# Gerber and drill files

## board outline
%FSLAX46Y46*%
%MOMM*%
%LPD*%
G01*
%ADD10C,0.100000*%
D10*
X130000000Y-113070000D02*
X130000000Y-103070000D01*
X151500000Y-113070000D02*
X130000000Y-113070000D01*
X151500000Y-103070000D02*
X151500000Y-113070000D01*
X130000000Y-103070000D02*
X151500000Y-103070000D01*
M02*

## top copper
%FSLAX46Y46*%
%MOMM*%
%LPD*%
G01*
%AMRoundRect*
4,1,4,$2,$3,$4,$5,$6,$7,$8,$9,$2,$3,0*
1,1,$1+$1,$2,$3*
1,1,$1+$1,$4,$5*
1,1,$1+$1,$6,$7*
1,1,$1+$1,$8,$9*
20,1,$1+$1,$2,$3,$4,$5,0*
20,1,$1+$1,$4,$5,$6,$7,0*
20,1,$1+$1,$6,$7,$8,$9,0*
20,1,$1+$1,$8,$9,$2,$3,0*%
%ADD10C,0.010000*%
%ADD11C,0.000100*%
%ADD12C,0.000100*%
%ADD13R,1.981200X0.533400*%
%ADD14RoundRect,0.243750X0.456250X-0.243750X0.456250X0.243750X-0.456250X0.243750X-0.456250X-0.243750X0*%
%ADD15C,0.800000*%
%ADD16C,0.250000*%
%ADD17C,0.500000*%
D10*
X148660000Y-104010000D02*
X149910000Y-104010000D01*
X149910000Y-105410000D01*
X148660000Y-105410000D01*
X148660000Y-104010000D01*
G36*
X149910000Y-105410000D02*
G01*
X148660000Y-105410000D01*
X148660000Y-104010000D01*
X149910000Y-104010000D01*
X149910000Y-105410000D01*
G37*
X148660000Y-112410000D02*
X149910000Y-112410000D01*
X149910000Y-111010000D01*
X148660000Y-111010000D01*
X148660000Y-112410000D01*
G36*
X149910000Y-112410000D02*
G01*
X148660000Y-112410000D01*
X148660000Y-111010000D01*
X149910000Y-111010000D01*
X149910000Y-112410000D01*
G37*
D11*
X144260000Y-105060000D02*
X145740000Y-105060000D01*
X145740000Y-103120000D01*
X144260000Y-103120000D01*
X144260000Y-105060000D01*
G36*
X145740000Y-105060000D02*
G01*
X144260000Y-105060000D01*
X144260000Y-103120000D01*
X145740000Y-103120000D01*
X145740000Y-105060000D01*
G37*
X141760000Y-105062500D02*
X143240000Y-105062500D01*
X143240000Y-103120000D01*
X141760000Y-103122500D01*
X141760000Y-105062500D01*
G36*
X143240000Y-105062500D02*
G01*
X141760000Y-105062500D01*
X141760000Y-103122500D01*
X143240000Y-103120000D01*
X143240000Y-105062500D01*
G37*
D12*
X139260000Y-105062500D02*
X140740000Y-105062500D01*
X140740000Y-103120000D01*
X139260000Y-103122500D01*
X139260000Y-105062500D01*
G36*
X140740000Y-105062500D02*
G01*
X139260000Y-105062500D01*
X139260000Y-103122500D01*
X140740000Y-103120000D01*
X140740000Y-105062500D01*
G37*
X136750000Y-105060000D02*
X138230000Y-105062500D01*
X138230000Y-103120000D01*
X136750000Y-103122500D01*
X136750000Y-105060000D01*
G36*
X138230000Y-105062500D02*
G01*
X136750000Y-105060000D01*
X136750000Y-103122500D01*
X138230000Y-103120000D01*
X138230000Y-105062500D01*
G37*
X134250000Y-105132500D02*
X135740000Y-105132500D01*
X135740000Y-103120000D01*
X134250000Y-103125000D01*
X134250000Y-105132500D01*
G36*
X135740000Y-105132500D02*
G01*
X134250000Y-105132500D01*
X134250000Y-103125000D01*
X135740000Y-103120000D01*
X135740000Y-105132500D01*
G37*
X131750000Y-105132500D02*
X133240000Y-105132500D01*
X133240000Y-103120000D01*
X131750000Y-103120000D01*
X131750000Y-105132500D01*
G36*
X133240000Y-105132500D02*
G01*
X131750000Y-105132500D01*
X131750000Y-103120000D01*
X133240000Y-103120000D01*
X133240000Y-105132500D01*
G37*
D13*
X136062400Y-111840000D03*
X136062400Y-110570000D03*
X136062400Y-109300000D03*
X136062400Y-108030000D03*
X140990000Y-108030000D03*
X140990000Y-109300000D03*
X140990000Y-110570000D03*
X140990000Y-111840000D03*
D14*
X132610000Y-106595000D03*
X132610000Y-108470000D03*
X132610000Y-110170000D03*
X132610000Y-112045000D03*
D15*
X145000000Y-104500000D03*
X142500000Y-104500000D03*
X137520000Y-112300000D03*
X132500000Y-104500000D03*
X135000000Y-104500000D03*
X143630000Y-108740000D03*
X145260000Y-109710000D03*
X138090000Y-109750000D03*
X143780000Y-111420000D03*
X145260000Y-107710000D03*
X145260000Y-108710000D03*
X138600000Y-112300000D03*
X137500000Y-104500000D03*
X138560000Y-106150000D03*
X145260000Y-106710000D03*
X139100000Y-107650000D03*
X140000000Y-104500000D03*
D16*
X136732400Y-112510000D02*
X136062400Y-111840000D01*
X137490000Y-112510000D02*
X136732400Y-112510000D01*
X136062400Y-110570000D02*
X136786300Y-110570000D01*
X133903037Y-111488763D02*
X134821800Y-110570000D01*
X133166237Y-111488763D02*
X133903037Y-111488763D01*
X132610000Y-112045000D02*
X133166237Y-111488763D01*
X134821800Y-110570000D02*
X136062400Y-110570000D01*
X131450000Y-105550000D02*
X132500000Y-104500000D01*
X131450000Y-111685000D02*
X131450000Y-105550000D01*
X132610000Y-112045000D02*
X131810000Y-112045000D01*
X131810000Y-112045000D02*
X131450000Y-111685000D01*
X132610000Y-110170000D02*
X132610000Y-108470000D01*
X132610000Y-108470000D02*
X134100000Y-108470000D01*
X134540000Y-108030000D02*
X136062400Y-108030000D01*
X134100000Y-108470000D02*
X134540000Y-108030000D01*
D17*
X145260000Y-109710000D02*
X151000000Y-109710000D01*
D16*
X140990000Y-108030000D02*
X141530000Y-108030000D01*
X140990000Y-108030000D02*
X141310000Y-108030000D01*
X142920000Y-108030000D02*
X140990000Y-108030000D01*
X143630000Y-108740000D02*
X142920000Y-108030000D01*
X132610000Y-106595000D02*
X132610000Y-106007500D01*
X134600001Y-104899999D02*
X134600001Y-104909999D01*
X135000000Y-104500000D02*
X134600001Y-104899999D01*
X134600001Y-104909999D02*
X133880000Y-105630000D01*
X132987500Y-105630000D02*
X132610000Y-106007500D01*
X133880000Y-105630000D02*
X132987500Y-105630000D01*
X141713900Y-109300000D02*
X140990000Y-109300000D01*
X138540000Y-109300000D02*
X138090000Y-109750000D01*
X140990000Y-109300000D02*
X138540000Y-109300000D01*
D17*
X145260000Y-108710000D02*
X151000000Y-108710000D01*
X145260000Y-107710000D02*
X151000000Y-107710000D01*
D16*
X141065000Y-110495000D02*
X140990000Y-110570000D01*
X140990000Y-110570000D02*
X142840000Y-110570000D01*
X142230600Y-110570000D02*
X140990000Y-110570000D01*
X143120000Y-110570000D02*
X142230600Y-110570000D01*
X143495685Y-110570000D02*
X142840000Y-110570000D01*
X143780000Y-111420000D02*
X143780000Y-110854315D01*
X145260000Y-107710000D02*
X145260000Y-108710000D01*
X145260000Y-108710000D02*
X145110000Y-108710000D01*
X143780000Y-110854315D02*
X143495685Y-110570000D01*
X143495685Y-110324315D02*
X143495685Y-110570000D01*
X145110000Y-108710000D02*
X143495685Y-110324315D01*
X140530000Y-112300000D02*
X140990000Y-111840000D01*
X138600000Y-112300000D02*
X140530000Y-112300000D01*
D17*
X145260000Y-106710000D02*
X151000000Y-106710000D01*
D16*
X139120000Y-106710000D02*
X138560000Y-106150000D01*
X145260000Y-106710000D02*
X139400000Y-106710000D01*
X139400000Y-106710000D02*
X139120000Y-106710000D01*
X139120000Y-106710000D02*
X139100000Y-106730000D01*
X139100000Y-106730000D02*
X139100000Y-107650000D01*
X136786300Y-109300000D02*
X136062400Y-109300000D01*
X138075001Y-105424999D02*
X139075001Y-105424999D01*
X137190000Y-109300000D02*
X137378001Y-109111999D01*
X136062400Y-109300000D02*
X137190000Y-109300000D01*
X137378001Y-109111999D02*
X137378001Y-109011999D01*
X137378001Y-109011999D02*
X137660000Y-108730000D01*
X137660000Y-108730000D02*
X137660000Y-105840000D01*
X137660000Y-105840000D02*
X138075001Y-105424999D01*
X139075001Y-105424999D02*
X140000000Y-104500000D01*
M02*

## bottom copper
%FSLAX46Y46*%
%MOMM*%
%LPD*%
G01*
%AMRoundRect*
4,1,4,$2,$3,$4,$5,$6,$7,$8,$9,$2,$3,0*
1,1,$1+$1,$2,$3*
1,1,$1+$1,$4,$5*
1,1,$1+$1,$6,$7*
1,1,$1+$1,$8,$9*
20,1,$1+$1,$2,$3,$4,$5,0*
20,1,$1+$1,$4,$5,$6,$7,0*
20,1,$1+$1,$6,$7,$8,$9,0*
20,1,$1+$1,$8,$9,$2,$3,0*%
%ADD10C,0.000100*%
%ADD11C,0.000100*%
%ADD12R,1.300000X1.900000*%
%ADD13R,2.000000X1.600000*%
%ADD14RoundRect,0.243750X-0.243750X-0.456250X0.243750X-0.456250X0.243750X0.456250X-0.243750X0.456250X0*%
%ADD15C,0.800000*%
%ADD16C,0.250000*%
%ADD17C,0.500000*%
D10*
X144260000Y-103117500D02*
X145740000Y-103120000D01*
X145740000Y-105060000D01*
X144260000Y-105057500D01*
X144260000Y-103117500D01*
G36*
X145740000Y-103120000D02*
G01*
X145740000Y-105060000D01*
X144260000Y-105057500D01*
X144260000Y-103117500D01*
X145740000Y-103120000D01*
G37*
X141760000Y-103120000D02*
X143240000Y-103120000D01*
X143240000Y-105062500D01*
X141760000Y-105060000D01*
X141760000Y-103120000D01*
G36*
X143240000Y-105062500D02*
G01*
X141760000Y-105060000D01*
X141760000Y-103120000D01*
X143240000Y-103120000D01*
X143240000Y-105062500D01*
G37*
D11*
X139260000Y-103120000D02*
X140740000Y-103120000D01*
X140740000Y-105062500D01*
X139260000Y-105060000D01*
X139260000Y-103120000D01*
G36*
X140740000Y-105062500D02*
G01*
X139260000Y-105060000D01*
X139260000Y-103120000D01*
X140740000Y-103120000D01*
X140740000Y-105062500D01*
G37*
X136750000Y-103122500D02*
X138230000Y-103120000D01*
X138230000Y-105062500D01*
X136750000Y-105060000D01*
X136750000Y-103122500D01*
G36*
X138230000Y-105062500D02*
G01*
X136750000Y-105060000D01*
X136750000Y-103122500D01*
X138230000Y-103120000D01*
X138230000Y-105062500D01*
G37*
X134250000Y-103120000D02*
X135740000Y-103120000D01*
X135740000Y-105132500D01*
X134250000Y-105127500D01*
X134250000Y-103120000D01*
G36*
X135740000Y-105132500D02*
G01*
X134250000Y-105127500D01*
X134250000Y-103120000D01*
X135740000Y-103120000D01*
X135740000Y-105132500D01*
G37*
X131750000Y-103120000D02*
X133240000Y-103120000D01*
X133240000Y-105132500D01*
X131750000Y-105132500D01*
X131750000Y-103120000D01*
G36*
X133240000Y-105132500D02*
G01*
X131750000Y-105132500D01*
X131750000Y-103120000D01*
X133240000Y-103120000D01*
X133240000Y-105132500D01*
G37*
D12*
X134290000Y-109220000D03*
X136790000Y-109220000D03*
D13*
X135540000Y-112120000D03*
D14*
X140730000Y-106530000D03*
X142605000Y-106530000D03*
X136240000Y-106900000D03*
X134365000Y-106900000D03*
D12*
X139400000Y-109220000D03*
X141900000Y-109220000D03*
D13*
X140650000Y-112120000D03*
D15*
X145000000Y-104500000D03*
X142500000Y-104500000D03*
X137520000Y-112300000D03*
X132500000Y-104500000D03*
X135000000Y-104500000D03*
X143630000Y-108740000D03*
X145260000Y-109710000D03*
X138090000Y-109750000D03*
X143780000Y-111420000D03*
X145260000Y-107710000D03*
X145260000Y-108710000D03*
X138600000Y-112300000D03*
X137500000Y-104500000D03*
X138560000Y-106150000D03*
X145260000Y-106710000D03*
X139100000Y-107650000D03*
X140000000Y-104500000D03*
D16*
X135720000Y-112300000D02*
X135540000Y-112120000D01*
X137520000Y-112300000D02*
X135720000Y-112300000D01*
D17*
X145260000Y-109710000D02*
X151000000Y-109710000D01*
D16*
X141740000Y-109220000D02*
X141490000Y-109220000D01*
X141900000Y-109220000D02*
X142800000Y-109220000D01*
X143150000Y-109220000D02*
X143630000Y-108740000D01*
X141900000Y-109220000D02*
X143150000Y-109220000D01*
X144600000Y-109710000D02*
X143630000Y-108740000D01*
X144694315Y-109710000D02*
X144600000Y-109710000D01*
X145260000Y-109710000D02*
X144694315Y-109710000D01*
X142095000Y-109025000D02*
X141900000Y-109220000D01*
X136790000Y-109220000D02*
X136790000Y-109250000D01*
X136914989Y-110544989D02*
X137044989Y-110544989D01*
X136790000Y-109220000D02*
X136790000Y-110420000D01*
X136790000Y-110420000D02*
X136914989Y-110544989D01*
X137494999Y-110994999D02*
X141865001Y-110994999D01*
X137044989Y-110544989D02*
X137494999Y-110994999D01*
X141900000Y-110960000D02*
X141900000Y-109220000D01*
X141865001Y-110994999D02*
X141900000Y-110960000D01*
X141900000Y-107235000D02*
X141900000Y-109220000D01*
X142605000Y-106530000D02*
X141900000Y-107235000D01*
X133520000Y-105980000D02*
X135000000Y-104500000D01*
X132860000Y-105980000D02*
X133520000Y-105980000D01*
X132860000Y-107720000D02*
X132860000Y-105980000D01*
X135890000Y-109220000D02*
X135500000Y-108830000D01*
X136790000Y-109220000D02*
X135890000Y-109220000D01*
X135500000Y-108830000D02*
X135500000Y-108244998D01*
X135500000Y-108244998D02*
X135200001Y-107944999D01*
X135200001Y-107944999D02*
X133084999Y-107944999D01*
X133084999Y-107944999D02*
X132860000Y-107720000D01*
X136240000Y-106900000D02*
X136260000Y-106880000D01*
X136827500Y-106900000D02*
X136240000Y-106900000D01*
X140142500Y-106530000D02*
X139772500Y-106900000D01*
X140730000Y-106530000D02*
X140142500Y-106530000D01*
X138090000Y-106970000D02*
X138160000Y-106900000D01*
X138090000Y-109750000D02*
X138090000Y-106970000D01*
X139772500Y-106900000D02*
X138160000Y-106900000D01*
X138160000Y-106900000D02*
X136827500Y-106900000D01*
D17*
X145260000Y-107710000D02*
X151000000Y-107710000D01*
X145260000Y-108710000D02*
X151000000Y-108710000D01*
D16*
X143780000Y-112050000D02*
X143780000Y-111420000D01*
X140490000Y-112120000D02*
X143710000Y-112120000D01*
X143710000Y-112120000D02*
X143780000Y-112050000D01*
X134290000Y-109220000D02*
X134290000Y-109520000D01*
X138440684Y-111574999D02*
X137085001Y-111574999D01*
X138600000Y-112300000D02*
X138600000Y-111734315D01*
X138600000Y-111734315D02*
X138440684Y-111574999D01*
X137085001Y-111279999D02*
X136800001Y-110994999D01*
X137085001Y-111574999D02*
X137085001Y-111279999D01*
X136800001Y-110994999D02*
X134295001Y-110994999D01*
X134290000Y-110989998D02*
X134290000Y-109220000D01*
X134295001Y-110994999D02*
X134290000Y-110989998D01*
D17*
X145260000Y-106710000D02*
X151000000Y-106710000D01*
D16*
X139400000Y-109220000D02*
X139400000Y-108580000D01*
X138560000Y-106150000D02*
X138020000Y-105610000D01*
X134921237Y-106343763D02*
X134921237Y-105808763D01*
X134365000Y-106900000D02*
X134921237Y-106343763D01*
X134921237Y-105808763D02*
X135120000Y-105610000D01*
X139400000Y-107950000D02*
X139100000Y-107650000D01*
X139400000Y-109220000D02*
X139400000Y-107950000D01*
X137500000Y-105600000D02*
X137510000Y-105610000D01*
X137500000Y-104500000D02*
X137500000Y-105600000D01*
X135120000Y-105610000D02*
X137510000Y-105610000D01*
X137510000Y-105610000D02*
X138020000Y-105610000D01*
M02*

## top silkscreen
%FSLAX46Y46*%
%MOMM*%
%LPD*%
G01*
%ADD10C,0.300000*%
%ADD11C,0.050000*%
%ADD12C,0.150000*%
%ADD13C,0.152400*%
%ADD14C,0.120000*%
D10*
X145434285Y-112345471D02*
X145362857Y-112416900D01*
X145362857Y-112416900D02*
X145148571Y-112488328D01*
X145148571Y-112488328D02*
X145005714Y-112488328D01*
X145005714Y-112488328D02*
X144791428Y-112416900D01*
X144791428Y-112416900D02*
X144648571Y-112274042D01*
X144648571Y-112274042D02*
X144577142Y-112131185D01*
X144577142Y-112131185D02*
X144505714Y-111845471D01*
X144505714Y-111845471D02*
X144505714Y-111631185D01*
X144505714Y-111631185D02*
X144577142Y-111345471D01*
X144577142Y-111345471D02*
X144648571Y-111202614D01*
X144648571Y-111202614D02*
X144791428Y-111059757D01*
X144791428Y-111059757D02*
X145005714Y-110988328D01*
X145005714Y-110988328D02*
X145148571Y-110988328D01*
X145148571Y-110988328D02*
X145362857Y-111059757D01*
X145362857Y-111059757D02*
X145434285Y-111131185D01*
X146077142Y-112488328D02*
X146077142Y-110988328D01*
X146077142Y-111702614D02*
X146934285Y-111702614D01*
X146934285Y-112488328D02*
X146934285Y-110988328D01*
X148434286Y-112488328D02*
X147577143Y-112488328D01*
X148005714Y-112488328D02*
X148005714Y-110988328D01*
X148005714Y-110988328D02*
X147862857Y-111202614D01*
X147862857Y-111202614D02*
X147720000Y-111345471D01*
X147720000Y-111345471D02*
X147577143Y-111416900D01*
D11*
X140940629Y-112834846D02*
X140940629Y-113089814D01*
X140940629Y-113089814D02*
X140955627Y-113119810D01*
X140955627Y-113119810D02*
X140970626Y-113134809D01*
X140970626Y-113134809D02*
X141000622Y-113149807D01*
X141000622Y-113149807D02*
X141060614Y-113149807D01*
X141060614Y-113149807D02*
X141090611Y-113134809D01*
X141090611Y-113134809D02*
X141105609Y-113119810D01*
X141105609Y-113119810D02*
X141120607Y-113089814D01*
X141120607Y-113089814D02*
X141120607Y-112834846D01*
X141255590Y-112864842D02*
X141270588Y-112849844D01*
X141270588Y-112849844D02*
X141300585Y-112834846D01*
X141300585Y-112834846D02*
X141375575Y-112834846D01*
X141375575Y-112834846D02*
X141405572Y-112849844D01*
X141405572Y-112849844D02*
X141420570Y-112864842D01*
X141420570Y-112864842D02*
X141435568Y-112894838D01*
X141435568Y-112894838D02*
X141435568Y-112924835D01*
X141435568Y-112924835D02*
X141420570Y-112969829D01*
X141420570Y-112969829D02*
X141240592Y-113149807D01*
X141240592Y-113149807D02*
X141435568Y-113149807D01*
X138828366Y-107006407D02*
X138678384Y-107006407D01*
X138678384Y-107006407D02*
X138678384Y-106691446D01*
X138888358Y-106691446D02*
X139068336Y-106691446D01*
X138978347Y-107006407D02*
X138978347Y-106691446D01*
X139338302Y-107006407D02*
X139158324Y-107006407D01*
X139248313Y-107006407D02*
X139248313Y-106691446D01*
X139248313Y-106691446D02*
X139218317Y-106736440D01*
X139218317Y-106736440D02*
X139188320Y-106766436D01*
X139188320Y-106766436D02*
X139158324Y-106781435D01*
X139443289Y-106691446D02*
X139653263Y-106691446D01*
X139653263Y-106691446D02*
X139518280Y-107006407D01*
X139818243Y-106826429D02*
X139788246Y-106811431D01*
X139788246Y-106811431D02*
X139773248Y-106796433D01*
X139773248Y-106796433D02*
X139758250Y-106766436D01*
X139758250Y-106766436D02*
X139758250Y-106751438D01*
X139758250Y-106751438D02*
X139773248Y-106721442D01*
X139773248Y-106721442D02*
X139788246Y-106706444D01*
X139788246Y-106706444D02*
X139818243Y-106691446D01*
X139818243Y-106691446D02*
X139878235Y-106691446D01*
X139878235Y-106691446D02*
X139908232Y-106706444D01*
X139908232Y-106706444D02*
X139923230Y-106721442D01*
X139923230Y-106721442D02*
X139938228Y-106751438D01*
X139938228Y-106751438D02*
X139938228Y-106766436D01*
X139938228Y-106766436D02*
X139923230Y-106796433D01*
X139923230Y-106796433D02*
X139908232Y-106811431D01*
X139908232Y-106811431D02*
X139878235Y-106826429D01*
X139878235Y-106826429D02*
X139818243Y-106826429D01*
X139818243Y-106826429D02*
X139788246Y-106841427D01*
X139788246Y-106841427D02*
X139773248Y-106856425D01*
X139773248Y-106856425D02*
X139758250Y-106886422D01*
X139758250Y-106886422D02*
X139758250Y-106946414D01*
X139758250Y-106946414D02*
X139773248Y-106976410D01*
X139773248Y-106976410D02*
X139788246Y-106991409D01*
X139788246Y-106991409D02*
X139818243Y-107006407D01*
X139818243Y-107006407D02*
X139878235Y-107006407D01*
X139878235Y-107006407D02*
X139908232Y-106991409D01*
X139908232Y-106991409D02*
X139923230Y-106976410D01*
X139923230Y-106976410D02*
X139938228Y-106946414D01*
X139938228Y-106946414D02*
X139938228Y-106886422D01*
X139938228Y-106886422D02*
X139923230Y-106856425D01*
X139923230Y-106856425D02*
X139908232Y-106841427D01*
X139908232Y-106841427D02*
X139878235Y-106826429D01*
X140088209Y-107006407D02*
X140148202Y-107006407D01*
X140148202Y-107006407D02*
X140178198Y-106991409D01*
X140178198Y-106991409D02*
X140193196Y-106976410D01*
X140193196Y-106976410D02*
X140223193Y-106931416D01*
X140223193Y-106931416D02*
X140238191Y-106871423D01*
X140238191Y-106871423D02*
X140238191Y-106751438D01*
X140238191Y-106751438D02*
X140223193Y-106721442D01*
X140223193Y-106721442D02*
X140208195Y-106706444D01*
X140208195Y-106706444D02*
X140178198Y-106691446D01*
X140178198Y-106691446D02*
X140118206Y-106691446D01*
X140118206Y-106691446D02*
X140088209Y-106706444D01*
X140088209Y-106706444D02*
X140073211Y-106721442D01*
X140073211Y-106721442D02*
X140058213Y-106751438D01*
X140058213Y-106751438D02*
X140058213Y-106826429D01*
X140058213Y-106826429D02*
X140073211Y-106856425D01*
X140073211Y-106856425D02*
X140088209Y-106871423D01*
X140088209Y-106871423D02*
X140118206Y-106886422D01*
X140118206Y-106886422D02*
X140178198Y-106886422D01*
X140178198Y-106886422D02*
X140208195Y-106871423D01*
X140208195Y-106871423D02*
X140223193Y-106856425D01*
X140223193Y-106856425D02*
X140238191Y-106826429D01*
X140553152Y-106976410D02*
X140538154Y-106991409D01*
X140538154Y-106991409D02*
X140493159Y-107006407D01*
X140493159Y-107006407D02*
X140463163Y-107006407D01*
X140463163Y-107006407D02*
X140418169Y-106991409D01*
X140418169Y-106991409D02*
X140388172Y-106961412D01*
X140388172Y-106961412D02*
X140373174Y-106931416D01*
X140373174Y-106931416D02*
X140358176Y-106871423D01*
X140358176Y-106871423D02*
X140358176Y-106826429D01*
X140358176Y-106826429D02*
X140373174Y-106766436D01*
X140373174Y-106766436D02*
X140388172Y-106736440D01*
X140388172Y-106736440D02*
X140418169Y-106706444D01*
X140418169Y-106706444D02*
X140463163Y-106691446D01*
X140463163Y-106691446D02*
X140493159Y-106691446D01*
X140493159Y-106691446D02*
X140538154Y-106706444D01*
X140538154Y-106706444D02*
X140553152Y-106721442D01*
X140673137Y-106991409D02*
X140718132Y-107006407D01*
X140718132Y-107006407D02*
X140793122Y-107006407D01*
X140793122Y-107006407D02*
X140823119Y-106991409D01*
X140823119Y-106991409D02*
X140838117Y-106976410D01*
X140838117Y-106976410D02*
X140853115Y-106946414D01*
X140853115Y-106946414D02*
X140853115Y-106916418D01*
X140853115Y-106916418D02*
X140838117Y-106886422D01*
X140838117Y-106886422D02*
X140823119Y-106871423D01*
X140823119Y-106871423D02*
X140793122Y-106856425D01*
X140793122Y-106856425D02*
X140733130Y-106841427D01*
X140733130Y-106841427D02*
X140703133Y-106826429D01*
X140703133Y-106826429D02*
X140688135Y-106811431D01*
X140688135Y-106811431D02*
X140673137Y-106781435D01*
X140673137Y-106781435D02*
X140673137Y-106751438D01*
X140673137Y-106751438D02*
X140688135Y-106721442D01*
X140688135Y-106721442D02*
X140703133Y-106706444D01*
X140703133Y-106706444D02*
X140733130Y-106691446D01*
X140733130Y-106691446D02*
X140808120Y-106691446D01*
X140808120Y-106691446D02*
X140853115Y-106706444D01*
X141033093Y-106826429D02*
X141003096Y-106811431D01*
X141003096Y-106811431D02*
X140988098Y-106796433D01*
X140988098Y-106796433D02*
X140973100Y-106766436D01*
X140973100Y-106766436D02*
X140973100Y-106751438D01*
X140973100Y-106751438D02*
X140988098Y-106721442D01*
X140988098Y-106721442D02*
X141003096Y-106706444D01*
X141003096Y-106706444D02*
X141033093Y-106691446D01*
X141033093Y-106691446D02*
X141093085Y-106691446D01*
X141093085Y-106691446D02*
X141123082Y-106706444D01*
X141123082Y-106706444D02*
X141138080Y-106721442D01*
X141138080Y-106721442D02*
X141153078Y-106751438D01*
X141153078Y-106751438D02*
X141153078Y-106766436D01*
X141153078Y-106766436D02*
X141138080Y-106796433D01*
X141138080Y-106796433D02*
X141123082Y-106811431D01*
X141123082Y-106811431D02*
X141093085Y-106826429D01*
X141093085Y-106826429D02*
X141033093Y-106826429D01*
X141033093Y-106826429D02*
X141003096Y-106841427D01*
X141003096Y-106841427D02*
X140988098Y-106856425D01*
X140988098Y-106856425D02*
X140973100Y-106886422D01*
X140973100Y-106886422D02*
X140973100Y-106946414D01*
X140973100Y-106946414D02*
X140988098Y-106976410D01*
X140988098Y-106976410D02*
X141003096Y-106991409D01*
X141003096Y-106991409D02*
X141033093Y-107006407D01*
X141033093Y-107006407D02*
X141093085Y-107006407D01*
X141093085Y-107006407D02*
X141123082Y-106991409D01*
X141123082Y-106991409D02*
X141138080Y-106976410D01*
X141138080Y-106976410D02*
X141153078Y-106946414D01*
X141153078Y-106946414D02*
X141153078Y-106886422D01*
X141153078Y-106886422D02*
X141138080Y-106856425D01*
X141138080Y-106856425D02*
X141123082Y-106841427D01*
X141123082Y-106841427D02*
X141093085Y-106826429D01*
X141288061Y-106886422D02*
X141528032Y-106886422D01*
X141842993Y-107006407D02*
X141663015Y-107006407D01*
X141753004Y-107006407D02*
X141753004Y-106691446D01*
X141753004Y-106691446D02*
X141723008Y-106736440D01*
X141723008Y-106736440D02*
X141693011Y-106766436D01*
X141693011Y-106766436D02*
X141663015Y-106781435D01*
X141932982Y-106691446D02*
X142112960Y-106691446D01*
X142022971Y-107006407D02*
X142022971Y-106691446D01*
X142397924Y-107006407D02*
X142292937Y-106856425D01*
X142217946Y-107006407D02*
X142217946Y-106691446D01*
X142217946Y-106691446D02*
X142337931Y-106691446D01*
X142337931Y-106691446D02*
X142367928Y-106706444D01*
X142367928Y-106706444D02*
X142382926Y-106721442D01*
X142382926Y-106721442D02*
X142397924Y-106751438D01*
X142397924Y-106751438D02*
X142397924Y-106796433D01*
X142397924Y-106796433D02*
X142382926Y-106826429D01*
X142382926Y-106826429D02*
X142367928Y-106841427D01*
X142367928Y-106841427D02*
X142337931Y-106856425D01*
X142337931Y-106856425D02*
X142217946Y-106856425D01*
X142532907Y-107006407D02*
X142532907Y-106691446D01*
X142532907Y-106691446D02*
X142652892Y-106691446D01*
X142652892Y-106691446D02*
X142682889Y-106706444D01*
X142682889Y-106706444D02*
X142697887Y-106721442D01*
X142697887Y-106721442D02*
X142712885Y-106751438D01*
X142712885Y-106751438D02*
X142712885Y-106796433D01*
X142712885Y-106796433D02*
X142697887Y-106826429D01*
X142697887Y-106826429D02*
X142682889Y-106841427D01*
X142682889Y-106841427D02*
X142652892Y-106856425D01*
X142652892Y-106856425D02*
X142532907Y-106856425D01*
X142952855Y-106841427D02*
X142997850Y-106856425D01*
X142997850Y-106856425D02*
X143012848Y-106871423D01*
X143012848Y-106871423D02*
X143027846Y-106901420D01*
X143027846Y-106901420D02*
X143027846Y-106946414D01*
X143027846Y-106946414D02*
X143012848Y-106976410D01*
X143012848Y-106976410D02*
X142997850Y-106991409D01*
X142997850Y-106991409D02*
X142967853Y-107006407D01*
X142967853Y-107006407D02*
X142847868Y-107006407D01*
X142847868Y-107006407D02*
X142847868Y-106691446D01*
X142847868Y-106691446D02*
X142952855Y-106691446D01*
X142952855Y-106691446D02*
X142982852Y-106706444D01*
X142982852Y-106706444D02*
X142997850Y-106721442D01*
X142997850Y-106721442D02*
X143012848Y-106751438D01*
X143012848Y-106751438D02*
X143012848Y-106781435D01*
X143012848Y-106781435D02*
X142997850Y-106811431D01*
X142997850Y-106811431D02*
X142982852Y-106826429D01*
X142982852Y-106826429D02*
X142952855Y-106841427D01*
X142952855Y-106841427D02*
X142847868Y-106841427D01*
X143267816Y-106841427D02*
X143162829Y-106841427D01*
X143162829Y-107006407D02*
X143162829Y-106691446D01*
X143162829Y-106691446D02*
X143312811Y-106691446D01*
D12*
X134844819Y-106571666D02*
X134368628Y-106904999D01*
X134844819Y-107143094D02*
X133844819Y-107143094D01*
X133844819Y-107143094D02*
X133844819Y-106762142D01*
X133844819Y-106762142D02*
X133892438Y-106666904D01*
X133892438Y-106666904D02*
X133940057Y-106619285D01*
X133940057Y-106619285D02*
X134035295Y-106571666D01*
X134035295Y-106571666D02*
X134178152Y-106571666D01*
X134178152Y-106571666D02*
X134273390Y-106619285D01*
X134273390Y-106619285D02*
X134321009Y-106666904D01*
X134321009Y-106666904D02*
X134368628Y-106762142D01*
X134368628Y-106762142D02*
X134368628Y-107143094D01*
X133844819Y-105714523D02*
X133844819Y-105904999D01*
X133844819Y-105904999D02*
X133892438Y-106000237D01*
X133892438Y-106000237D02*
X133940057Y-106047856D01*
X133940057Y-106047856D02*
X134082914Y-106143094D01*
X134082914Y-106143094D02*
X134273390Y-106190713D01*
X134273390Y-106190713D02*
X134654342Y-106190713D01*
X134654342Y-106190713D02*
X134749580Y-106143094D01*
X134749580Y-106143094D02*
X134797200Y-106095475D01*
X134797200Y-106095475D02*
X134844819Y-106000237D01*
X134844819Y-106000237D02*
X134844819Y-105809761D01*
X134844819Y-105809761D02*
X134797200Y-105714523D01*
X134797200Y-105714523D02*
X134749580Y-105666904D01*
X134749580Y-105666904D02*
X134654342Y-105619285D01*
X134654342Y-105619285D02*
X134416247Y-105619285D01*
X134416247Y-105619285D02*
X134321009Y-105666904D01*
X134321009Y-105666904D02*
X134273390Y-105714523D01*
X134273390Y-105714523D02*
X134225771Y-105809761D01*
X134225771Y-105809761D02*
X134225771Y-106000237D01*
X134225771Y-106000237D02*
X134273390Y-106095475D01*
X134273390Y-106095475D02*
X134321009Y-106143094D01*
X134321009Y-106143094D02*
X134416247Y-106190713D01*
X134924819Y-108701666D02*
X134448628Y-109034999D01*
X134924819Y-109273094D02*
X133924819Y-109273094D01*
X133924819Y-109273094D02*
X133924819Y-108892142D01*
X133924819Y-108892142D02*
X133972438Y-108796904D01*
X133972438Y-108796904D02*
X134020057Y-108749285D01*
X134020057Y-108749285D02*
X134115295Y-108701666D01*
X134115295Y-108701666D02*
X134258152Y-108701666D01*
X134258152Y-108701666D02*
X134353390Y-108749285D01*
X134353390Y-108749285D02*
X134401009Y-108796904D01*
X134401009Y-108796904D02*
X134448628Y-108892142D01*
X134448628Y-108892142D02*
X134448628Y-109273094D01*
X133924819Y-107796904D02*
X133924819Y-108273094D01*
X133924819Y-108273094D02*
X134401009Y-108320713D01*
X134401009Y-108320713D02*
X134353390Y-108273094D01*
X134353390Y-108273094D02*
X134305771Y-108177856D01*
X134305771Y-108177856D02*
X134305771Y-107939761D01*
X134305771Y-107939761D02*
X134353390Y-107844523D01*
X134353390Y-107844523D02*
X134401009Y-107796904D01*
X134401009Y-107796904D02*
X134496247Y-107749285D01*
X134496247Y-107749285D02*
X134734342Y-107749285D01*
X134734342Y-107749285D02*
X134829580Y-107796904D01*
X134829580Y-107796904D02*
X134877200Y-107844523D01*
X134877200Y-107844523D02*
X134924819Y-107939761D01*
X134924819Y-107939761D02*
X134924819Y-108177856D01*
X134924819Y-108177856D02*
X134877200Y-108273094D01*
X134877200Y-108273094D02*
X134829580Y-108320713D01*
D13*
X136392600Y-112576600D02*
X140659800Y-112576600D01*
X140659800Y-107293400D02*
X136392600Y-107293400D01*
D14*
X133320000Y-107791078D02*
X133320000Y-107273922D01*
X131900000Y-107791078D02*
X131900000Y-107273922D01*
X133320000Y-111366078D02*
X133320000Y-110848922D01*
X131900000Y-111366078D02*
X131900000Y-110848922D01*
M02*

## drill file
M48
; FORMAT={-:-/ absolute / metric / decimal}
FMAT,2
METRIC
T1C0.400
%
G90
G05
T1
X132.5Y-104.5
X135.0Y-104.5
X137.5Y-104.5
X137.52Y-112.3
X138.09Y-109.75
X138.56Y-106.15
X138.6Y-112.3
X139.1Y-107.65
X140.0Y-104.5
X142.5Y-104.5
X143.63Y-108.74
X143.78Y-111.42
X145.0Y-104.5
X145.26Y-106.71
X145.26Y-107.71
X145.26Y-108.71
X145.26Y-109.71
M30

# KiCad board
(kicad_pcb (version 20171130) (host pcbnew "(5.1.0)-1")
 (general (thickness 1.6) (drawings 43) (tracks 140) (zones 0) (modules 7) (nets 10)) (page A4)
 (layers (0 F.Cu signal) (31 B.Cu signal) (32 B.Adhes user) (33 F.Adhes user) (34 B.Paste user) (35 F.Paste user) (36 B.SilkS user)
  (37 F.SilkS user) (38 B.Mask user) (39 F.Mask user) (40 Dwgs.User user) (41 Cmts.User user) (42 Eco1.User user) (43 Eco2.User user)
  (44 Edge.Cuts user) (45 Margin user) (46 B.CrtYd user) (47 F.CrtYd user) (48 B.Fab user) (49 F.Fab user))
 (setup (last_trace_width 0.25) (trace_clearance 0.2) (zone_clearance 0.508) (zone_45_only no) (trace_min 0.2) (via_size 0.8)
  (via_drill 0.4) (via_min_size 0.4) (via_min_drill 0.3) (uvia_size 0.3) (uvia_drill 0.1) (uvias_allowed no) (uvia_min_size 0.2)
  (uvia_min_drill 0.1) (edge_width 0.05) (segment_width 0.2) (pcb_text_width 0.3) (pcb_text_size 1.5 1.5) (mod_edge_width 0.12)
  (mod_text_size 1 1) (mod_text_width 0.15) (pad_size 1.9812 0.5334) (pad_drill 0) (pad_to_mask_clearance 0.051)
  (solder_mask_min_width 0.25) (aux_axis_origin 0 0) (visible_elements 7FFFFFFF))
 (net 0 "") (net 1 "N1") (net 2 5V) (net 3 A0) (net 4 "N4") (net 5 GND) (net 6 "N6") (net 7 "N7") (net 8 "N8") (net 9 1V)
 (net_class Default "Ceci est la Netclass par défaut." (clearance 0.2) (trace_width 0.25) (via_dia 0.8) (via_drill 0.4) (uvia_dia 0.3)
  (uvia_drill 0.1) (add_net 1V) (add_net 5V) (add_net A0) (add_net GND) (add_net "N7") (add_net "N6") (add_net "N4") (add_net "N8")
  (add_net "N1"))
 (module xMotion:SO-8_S (layer F.Cu) (at 138.5262 109.935 180)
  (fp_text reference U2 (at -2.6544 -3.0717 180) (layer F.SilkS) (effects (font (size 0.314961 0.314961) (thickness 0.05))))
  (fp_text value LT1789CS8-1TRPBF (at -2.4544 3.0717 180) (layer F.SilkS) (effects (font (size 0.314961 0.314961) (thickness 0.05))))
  (fp_line (start 2.1336 -2.6416) (end -2.1336 -2.6416) (layer F.SilkS) (width 0.1524))
  (fp_line (start -2.1336 2.6416) (end 2.1336 2.6416) (layer F.SilkS) (width 0.1524))
  (pad 8 smd rect (at 2.4638 -1.905 180) (size 1.9812 0.5334) (layers F.Cu F.Paste F.Mask) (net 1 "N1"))
  (pad 7 smd rect (at 2.4638 -0.635 180) (size 1.9812 0.5334) (layers F.Cu F.Paste F.Mask) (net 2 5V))
  (pad 6 smd rect (at 2.4638 0.635 180) (size 1.9812 0.5334) (layers F.Cu F.Paste F.Mask) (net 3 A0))
  (pad 5 smd rect (at 2.4638 1.905 180) (size 1.9812 0.5334) (layers F.Cu F.Paste F.Mask) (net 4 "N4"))
  (pad 4 smd rect (at -2.4638 1.905 180) (size 1.9812 0.5334) (layers F.Cu F.Paste F.Mask) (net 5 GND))
  (pad 3 smd rect (at -2.4638 0.635 180) (size 1.9812 0.5334) (layers F.Cu F.Paste F.Mask) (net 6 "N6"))
  (pad 2 smd rect (at -2.4638 -0.635 180) (size 1.9812 0.5334) (layers F.Cu F.Paste F.Mask) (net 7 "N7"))
  (pad 1 smd rect (at -2.4638 -1.905 180) (size 1.9812 0.5334) (layers F.Cu F.Paste F.Mask) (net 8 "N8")))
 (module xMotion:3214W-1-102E (layer B.Cu) (at 135.54 112.12 90)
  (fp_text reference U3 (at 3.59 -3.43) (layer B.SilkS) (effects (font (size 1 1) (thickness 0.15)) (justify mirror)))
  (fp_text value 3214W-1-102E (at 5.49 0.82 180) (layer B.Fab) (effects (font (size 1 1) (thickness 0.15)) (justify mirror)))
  (pad 3 smd rect (at 2.9 -1.25 90) (size 1.9 1.3) (layers B.Cu B.Paste B.Mask) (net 8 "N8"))
  (pad 2 smd rect (at 2.9 1.25 90) (size 1.9 1.3) (layers B.Cu B.Paste B.Mask) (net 5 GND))
  (pad 1 smd rect (at 0 0 90) (size 1.6 2) (layers B.Cu B.Paste B.Mask) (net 1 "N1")))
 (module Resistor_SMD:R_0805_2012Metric (layer F.Cu) (at 132.61 107.5325 90)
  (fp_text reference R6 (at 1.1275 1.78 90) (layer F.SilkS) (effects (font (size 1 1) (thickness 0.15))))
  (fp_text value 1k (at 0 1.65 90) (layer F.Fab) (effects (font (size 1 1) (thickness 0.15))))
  (fp_line (start -0.258578 0.71) (end 0.258578 0.71) (layer F.SilkS) (width 0.12))
  (fp_line (start -0.258578 -0.71) (end 0.258578 -0.71) (layer F.SilkS) (width 0.12))
  (pad 2 smd roundrect (at 0.9375 0 90) (size 0.975 1.4) (layers F.Cu F.Paste F.Mask) (roundrect_rratio 0.25) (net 5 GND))
  (pad 1 smd roundrect (at -0.9375 0 90) (size 0.975 1.4) (layers F.Cu F.Paste F.Mask) (roundrect_rratio 0.25) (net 4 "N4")))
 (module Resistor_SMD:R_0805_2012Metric (layer F.Cu) (at 132.61 111.1075 90)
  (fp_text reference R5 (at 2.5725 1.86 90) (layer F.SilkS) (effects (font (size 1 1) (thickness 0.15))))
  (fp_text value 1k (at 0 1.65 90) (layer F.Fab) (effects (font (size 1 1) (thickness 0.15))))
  (fp_line (start -0.258578 0.71) (end 0.258578 0.71) (layer F.SilkS) (width 0.12))
  (fp_line (start -0.258578 -0.71) (end 0.258578 -0.71) (layer F.SilkS) (width 0.12))
  (pad 2 smd roundrect (at 0.9375 0 90) (size 0.975 1.4) (layers F.Cu F.Paste F.Mask) (roundrect_rratio 0.25) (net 4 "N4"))
  (pad 1 smd roundrect (at -0.9375 0 90) (size 0.975 1.4) (layers F.Cu F.Paste F.Mask) (roundrect_rratio 0.25) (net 2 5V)))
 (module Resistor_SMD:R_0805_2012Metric (layer B.Cu) (at 141.6675 106.53)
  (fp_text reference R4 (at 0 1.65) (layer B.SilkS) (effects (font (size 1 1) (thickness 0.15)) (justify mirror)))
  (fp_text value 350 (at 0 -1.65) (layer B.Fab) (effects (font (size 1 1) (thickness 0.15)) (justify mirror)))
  (pad 1 smd roundrect (at -0.9375 0) (size 0.975 1.4) (layers B.Cu B.Paste B.Mask) (roundrect_rratio 0.25) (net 6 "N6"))
  (pad 2 smd roundrect (at 0.9375 0) (size 0.975 1.4) (layers B.Cu B.Paste B.Mask) (roundrect_rratio 0.25) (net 5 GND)))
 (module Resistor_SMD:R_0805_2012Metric (layer B.Cu) (at 135.3025 106.9)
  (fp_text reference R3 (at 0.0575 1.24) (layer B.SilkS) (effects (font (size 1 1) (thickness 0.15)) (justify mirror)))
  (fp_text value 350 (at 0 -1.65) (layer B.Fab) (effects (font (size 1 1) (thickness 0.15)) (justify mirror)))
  (pad 2 smd roundrect (at 0.9375 0) (size 0.975 1.4) (layers B.Cu B.Paste B.Mask) (roundrect_rratio 0.25) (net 6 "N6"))
  (pad 1 smd roundrect (at -0.9375 0) (size 0.975 1.4) (layers B.Cu B.Paste B.Mask) (roundrect_rratio 0.25) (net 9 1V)))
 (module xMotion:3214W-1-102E (layer B.Cu) (at 140.65 112.12 90)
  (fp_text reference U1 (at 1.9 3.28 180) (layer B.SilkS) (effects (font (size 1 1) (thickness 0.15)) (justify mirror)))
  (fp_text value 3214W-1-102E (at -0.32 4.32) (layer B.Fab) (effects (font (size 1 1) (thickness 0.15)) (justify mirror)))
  (pad 3 smd rect (at 2.9 -1.25 90) (size 1.9 1.3) (layers B.Cu B.Paste B.Mask) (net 9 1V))
  (pad 2 smd rect (at 2.9 1.25 90) (size 1.9 1.3) (layers B.Cu B.Paste B.Mask) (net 5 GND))
  (pad 1 smd rect (at 0 0 90) (size 1.6 2) (layers B.Cu B.Paste B.Mask) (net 7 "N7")))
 (gr_poly (pts (xy 148.66 104.01) (xy 149.91 104.01) (xy 149.91 105.41) (xy 148.66 105.41)) (layer F.Cu) (width 0.01))
 (gr_poly (pts (xy 148.66 112.41) (xy 149.91 112.41) (xy 149.91 111.01) (xy 148.66 111.01)) (layer F.Cu) (width 0.01))
 (gr_poly (pts (xy 144.26 103.1175) (xy 145.74 103.12) (xy 145.74 105.06) (xy 144.26 105.0575)) (layer B.Cu) (width 0.0001))
 (gr_poly (pts (xy 144.26 105.06) (xy 145.74 105.06) (xy 145.74 103.12) (xy 144.26 103.12)) (layer F.Cu) (width 0.0001))
 (gr_poly (pts (xy 141.76 103.12) (xy 143.24 103.12) (xy 143.24 105.0625) (xy 141.76 105.06)) (layer B.Cu) (width 0.0001))
 (gr_poly (pts (xy 141.76 105.0625) (xy 143.24 105.0625) (xy 143.24 103.12) (xy 141.76 103.1225)) (layer F.Cu) (width 0.0001))
 (gr_poly (pts (xy 139.26 103.12) (xy 140.74 103.12) (xy 140.74 105.0625) (xy 139.26 105.06)) (layer B.Cu) (width 0.0001))
 (gr_poly (pts (xy 139.26 105.0625) (xy 140.74 105.0625) (xy 140.74 103.12) (xy 139.26 103.1225)) (layer F.Cu) (width 0.0001))
 (gr_poly (pts (xy 136.75 103.1225) (xy 138.23 103.12) (xy 138.23 105.0625) (xy 136.75 105.06)) (layer B.Cu) (width 0.0001))
 (gr_poly (pts (xy 136.75 105.06) (xy 138.23 105.0625) (xy 138.23 103.12) (xy 136.75 103.1225)) (layer F.Cu) (width 0.0001))
 (gr_poly (pts (xy 134.25 103.12) (xy 135.74 103.12) (xy 135.74 105.1325) (xy 134.25 105.1275)) (layer B.Cu) (width 0.0001))
 (gr_poly (pts (xy 134.25 105.1325) (xy 135.74 105.1325) (xy 135.74 103.12) (xy 134.25 103.125)) (layer F.Cu) (width 0.0001))
 (gr_poly (pts (xy 131.75 103.12) (xy 133.24 103.12) (xy 133.24 105.1325) (xy 131.75 105.1325)) (layer B.Cu) (width 0.0001))
 (gr_poly (pts (xy 131.75 105.1325) (xy 133.24 105.1325) (xy 133.24 103.12) (xy 131.75 103.12)) (layer F.Cu) (width 0.0001))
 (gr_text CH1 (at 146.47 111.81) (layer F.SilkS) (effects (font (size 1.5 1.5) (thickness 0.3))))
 (gr_line (start 130 113.07) (end 130 103.07) (layer Edge.Cuts) (width 0.1))
 (gr_line (start 151.5 113.07) (end 130 113.07) (layer Edge.Cuts) (width 0.1))
 (gr_line (start 151.5 103.07) (end 151.5 113.07) (layer Edge.Cuts) (width 0.1))
 (gr_line (start 130 103.07) (end 151.5 103.07) (layer Edge.Cuts) (width 0.1))
 (via (at 145 104.5) (size 0.8) (drill 0.4) (layers F.Cu B.Cu) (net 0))
 (via (at 142.5 104.5) (size 0.8) (drill 0.4) (layers F.Cu B.Cu) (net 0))
 (via (at 137.52 112.3) (size 0.8) (drill 0.4) (layers F.Cu B.Cu) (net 1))
 (segment (start 136.7324 112.51) (end 136.0624 111.84) (width 0.25) (layer F.Cu) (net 1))
 (segment (start 137.49 112.51) (end 136.7324 112.51) (width 0.25) (layer F.Cu) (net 1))
 (segment (start 135.72 112.3) (end 135.54 112.12) (width 0.25) (layer B.Cu) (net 1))
 (segment (start 137.52 112.3) (end 135.72 112.3) (width 0.25) (layer B.Cu) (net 1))
 (via (at 132.5 104.5) (size 0.8) (drill 0.4) (layers F.Cu B.Cu) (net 2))
 (segment (start 136.0624 110.57) (end 136.7863 110.57) (width 0.25) (layer F.Cu) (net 2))
 (segment (start 133.903037 111.488763) (end 134.8218 110.57) (width 0.25) (layer F.Cu) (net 2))
 (segment (start 133.166237 111.488763) (end 133.903037 111.488763) (width 0.25) (layer F.Cu) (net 2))
 (segment (start 132.61 112.045) (end 133.166237 111.488763) (width 0.25) (layer F.Cu) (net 2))
 (segment (start 134.8218 110.57) (end 136.0624 110.57) (width 0.25) (layer F.Cu) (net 2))
 (segment (start 131.45 105.55) (end 132.5 104.5) (width 0.25) (layer F.Cu) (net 2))
 (segment (start 131.45 111.685) (end 131.45 105.55) (width 0.25) (layer F.Cu) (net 2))
 (segment (start 132.61 112.045) (end 131.81 112.045) (width 0.25) (layer F.Cu) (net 2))
 (segment (start 131.81 112.045) (end 131.45 111.685) (width 0.25) (layer F.Cu) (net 2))
 (segment (start 132.61 110.17) (end 132.61 108.47) (width 0.25) (layer F.Cu) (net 4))
 (segment (start 132.61 108.47) (end 134.1 108.47) (width 0.25) (layer F.Cu) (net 4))
 (segment (start 134.54 108.03) (end 136.0624 108.03) (width 0.25) (layer F.Cu) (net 4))
 (segment (start 134.1 108.47) (end 134.54 108.03) (width 0.25) (layer F.Cu) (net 4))
 (via (at 135 104.5) (size 0.8) (drill 0.4) (layers F.Cu B.Cu) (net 5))
 (via (at 143.63 108.74) (size 0.8) (drill 0.4) (layers F.Cu B.Cu) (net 5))
 (segment (start 145.26 109.71) (end 151 109.71) (width 0.5) (layer F.Cu) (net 5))
 (segment (start 140.99 108.03) (end 141.53 108.03) (width 0.25) (layer F.Cu) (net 5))
 (segment (start 140.99 108.03) (end 141.31 108.03) (width 0.25) (layer F.Cu) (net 5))
 (segment (start 145.26 109.71) (end 151 109.71) (width 0.5) (layer B.Cu) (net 5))
 (via (at 145.26 109.71) (size 0.8) (drill 0.4) (layers F.Cu B.Cu) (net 5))
 (segment (start 141.74 109.22) (end 141.49 109.22) (width 0.25) (layer B.Cu) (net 5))
 (segment (start 141.9 109.22) (end 142.8 109.22) (width 0.25) (layer B.Cu) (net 5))
 (segment (start 142.92 108.03) (end 140.99 108.03) (width 0.25) (layer F.Cu) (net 5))
 (segment (start 143.63 108.74) (end 142.92 108.03) (width 0.25) (layer F.Cu) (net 5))
 (segment (start 143.15 109.22) (end 143.63 108.74) (width 0.25) (layer B.Cu) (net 5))
 (segment (start 141.9 109.22) (end 143.15 109.22) (width 0.25) (layer B.Cu) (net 5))
 (segment (start 144.6 109.71) (end 143.63 108.74) (width 0.25) (layer B.Cu) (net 5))
 (segment (start 144.694315 109.71) (end 144.6 109.71) (width 0.25) (layer B.Cu) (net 5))
 (segment (start 145.26 109.71) (end 144.694315 109.71) (width 0.25) (layer B.Cu) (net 5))
 (segment (start 142.095 109.025) (end 141.9 109.22) (width 0.25) (layer B.Cu) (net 5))
 (segment (start 136.79 109.22) (end 136.79 109.25) (width 0.25) (layer B.Cu) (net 5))
 (segment (start 136.914989 110.544989) (end 137.044989 110.544989) (width 0.25) (layer B.Cu) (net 5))
 (segment (start 136.79 109.22) (end 136.79 110.42) (width 0.25) (layer B.Cu) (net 5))
 (segment (start 136.79 110.42) (end 136.914989 110.544989) (width 0.25) (layer B.Cu) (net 5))
 (segment (start 137.494999 110.994999) (end 141.865001 110.994999) (width 0.25) (layer B.Cu) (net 5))
 (segment (start 137.044989 110.544989) (end 137.494999 110.994999) (width 0.25) (layer B.Cu) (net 5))
 (segment (start 141.9 110.96) (end 141.9 109.22) (width 0.25) (layer B.Cu) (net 5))
 (segment (start 141.865001 110.994999) (end 141.9 110.96) (width 0.25) (layer B.Cu) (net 5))
 (segment (start 141.9 107.235) (end 141.9 109.22) (width 0.25) (layer B.Cu) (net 5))
 (segment (start 142.605 106.53) (end 141.9 107.235) (width 0.25) (layer B.Cu) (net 5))
 (segment (start 132.61 106.595) (end 132.61 106.0075) (width 0.25) (layer F.Cu) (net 5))
 (segment (start 134.600001 104.899999) (end 134.600001 104.909999) (width 0.25) (layer F.Cu) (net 5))
 (segment (start 135 104.5) (end 134.600001 104.899999) (width 0.25) (layer F.Cu) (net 5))
 (segment (start 134.600001 104.909999) (end 133.88 105.63) (width 0.25) (layer F.Cu) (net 5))
 (segment (start 132.9875 105.63) (end 132.61 106.0075) (width 0.25) (layer F.Cu) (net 5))
 (segment (start 133.88 105.63) (end 132.9875 105.63) (width 0.25) (layer F.Cu) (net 5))
 (segment (start 133.52 105.98) (end 135 104.5) (width 0.25) (layer B.Cu) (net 5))
 (segment (start 132.86 105.98) (end 133.52 105.98) (width 0.25) (layer B.Cu) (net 5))
 (segment (start 132.86 107.72) (end 132.86 105.98) (width 0.25) (layer B.Cu) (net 5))
 (segment (start 135.89 109.22) (end 135.5 108.83) (width 0.25) (layer B.Cu) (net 5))
 (segment (start 136.79 109.22) (end 135.89 109.22) (width 0.25) (layer B.Cu) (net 5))
 (segment (start 135.5 108.83) (end 135.5 108.244998) (width 0.25) (layer B.Cu) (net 5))
 (segment (start 135.5 108.244998) (end 135.200001 107.944999) (width 0.25) (layer B.Cu) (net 5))
 (segment (start 135.200001 107.944999) (end 133.084999 107.944999) (width 0.25) (layer B.Cu) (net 5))
 (segment (start 133.084999 107.944999) (end 132.86 107.72) (width 0.25) (layer B.Cu) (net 5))
 (via (at 138.09 109.75) (size 0.8) (drill 0.4) (layers F.Cu B.Cu) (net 6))
 (segment (start 141.7139 109.3) (end 140.99 109.3) (width 0.25) (layer F.Cu) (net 6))
 (segment (start 136.24 106.9) (end 136.26 106.88) (width 0.25) (layer B.Cu) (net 6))
 (segment (start 136.8275 106.9) (end 136.24 106.9) (width 0.25) (layer B.Cu) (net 6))
 (segment (start 140.1425 106.53) (end 139.7725 106.9) (width 0.25) (layer B.Cu) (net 6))
 (segment (start 140.73 106.53) (end 140.1425 106.53) (width 0.25) (layer B.Cu) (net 6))
 (segment (start 138.54 109.3) (end 138.09 109.75) (width 0.25) (layer F.Cu) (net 6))
 (segment (start 140.99 109.3) (end 138.54 109.3) (width 0.25) (layer F.Cu) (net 6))
 (segment (start 138.09 106.97) (end 138.16 106.9) (width 0.25) (layer B.Cu) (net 6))
 (segment (start 138.09 109.75) (end 138.09 106.97) (width 0.25) (layer B.Cu) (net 6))
 (segment (start 139.7725 106.9) (end 138.16 106.9) (width 0.25) (layer B.Cu) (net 6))
 (segment (start 138.16 106.9) (end 136.8275 106.9) (width 0.25) (layer B.Cu) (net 6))
 (via (at 143.78 111.42) (size 0.8) (drill 0.4) (layers F.Cu B.Cu) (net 7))
 (segment (start 145.26 108.71) (end 151 108.71) (width 0.5) (layer F.Cu) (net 7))
 (segment (start 145.26 107.71) (end 151 107.71) (width 0.5) (layer F.Cu) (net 7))
 (segment (start 145.26 107.71) (end 151 107.71) (width 0.5) (layer B.Cu) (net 7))
 (segment (start 145.26 108.71) (end 151 108.71) (width 0.5) (layer B.Cu) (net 7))
 (via (at 145.26 107.71) (size 0.8) (drill 0.4) (layers F.Cu B.Cu) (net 7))
 (via (at 145.26 108.71) (size 0.8) (drill 0.4) (layers F.Cu B.Cu) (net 7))
 (segment (start 141.065 110.495) (end 140.99 110.57) (width 0.25) (layer F.Cu) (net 7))
 (segment (start 140.99 110.57) (end 142.84 110.57) (width 0.25) (layer F.Cu) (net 7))
 (segment (start 142.2306 110.57) (end 140.99 110.57) (width 0.25) (layer F.Cu) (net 7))
 (segment (start 143.12 110.57) (end 142.2306 110.57) (width 0.25) (layer F.Cu) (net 7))
 (segment (start 143.495685 110.57) (end 142.84 110.57) (width 0.25) (layer F.Cu) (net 7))
 (segment (start 143.78 111.42) (end 143.78 110.854315) (width 0.25) (layer F.Cu) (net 7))
 (segment (start 143.78 112.05) (end 143.78 111.42) (width 0.25) (layer B.Cu) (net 7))
 (segment (start 140.49 112.12) (end 143.71 112.12) (width 0.25) (layer B.Cu) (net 7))
 (segment (start 143.71 112.12) (end 143.78 112.05) (width 0.25) (layer B.Cu) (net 7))
 (segment (start 145.26 107.71) (end 145.26 108.71) (width 0.25) (layer F.Cu) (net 7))
 (segment (start 145.26 108.71) (end 145.11 108.71) (width 0.25) (layer F.Cu) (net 7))
 (segment (start 143.78 110.854315) (end 143.495685 110.57) (width 0.25) (layer F.Cu) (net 7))
 (segment (start 143.495685 110.324315) (end 143.495685 110.57) (width 0.25) (layer F.Cu) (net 7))
 (segment (start 145.11 108.71) (end 143.495685 110.324315) (width 0.25) (layer F.Cu) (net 7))
 (segment (start 134.29 109.22) (end 134.29 109.52) (width 0.25) (layer B.Cu) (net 8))
 (via (at 138.6 112.3) (size 0.8) (drill 0.4) (layers F.Cu B.Cu) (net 8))
 (segment (start 140.53 112.3) (end 140.99 111.84) (width 0.25) (layer F.Cu) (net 8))
 (segment (start 138.6 112.3) (end 140.53 112.3) (width 0.25) (layer F.Cu) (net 8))
 (segment (start 138.440684 111.574999) (end 137.085001 111.574999) (width 0.25) (layer B.Cu) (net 8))
 (segment (start 138.6 112.3) (end 138.6 111.734315) (width 0.25) (layer B.Cu) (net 8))
 (segment (start 138.6 111.734315) (end 138.440684 111.574999) (width 0.25) (layer B.Cu) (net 8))
 (segment (start 137.085001 111.279999) (end 136.800001 110.994999) (width 0.25) (layer B.Cu) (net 8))
 (segment (start 137.085001 111.574999) (end 137.085001 111.279999) (width 0.25) (layer B.Cu) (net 8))
 (segment (start 136.800001 110.994999) (end 134.295001 110.994999) (width 0.25) (layer B.Cu) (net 8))
 (segment (start 134.29 110.989998) (end 134.29 109.22) (width 0.25) (layer B.Cu) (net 8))
 (segment (start 134.295001 110.994999) (end 134.29 110.989998) (width 0.25) (layer B.Cu) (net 8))
 (via (at 137.5 104.5) (size 0.8) (drill 0.4) (layers F.Cu B.Cu) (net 9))
 (via (at 138.56 106.15) (size 0.8) (drill 0.4) (layers F.Cu B.Cu) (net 9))
 (segment (start 145.26 106.71) (end 151 106.71) (width 0.5) (layer B.Cu) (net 9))
 (segment (start 145.26 106.71) (end 151 106.71) (width 0.5) (layer F.Cu) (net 9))
 (via (at 145.26 106.71) (size 0.8) (drill 0.4) (layers F.Cu B.Cu) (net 9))
 (segment (start 139.4 109.22) (end 139.4 108.58) (width 0.25) (layer B.Cu) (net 9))
 (segment (start 138.56 106.15) (end 138.02 105.61) (width 0.25) (layer B.Cu) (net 9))
 (segment (start 134.921237 106.343763) (end 134.921237 105.808763) (width 0.25) (layer B.Cu) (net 9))
 (segment (start 134.365 106.9) (end 134.921237 106.343763) (width 0.25) (layer B.Cu) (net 9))
 (segment (start 134.921237 105.808763) (end 135.12 105.61) (width 0.25) (layer B.Cu) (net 9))
 (segment (start 139.12 106.71) (end 138.56 106.15) (width 0.25) (layer F.Cu) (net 9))
 (segment (start 145.26 106.71) (end 139.4 106.71) (width 0.25) (layer F.Cu) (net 9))
 (segment (start 139.4 106.71) (end 139.12 106.71) (width 0.25) (layer F.Cu) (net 9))
 (segment (start 139.4 107.95) (end 139.1 107.65) (width 0.25) (layer B.Cu) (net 9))
 (segment (start 139.4 109.22) (end 139.4 107.95) (width 0.25) (layer B.Cu) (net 9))
 (segment (start 139.12 106.71) (end 139.1 106.73) (width 0.25) (layer F.Cu) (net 9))
 (via (at 139.1 107.65) (size 0.8) (drill 0.4) (layers F.Cu B.Cu) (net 9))
 (segment (start 139.1 106.73) (end 139.1 107.65) (width 0.25) (layer F.Cu) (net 9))
 (segment (start 137.5 105.6) (end 137.51 105.61) (width 0.25) (layer B.Cu) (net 9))
 (segment (start 137.5 104.5) (end 137.5 105.6) (width 0.25) (layer B.Cu) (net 9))
 (segment (start 135.12 105.61) (end 137.51 105.61) (width 0.25) (layer B.Cu) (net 9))
 (segment (start 137.51 105.61) (end 138.02 105.61) (width 0.25) (layer B.Cu) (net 9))
 (via (at 140 104.5) (size 0.8) (drill 0.4) (layers F.Cu B.Cu) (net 3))
 (segment (start 136.7863 109.3) (end 136.0624 109.3) (width 0.25) (layer F.Cu) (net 3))
 (segment (start 138.075001 105.424999) (end 139.075001 105.424999) (width 0.25) (layer F.Cu) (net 3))
 (segment (start 137.19 109.3) (end 137.378001 109.111999) (width 0.25) (layer F.Cu) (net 3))
 (segment (start 136.0624 109.3) (end 137.19 109.3) (width 0.25) (layer F.Cu) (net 3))
 (segment (start 137.378001 109.111999) (end 137.378001 109.011999) (width 0.25) (layer F.Cu) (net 3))
 (segment (start 137.378001 109.011999) (end 137.66 108.73) (width 0.25) (layer F.Cu) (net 3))
 (segment (start 137.66 108.73) (end 137.66 105.84) (width 0.25) (layer F.Cu) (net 3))
 (segment (start 137.66 105.84) (end 138.075001 105.424999) (width 0.25) (layer F.Cu) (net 3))
 (segment (start 139.075001 105.424999) (end 140 104.5) (width 0.25) (layer F.Cu) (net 3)))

